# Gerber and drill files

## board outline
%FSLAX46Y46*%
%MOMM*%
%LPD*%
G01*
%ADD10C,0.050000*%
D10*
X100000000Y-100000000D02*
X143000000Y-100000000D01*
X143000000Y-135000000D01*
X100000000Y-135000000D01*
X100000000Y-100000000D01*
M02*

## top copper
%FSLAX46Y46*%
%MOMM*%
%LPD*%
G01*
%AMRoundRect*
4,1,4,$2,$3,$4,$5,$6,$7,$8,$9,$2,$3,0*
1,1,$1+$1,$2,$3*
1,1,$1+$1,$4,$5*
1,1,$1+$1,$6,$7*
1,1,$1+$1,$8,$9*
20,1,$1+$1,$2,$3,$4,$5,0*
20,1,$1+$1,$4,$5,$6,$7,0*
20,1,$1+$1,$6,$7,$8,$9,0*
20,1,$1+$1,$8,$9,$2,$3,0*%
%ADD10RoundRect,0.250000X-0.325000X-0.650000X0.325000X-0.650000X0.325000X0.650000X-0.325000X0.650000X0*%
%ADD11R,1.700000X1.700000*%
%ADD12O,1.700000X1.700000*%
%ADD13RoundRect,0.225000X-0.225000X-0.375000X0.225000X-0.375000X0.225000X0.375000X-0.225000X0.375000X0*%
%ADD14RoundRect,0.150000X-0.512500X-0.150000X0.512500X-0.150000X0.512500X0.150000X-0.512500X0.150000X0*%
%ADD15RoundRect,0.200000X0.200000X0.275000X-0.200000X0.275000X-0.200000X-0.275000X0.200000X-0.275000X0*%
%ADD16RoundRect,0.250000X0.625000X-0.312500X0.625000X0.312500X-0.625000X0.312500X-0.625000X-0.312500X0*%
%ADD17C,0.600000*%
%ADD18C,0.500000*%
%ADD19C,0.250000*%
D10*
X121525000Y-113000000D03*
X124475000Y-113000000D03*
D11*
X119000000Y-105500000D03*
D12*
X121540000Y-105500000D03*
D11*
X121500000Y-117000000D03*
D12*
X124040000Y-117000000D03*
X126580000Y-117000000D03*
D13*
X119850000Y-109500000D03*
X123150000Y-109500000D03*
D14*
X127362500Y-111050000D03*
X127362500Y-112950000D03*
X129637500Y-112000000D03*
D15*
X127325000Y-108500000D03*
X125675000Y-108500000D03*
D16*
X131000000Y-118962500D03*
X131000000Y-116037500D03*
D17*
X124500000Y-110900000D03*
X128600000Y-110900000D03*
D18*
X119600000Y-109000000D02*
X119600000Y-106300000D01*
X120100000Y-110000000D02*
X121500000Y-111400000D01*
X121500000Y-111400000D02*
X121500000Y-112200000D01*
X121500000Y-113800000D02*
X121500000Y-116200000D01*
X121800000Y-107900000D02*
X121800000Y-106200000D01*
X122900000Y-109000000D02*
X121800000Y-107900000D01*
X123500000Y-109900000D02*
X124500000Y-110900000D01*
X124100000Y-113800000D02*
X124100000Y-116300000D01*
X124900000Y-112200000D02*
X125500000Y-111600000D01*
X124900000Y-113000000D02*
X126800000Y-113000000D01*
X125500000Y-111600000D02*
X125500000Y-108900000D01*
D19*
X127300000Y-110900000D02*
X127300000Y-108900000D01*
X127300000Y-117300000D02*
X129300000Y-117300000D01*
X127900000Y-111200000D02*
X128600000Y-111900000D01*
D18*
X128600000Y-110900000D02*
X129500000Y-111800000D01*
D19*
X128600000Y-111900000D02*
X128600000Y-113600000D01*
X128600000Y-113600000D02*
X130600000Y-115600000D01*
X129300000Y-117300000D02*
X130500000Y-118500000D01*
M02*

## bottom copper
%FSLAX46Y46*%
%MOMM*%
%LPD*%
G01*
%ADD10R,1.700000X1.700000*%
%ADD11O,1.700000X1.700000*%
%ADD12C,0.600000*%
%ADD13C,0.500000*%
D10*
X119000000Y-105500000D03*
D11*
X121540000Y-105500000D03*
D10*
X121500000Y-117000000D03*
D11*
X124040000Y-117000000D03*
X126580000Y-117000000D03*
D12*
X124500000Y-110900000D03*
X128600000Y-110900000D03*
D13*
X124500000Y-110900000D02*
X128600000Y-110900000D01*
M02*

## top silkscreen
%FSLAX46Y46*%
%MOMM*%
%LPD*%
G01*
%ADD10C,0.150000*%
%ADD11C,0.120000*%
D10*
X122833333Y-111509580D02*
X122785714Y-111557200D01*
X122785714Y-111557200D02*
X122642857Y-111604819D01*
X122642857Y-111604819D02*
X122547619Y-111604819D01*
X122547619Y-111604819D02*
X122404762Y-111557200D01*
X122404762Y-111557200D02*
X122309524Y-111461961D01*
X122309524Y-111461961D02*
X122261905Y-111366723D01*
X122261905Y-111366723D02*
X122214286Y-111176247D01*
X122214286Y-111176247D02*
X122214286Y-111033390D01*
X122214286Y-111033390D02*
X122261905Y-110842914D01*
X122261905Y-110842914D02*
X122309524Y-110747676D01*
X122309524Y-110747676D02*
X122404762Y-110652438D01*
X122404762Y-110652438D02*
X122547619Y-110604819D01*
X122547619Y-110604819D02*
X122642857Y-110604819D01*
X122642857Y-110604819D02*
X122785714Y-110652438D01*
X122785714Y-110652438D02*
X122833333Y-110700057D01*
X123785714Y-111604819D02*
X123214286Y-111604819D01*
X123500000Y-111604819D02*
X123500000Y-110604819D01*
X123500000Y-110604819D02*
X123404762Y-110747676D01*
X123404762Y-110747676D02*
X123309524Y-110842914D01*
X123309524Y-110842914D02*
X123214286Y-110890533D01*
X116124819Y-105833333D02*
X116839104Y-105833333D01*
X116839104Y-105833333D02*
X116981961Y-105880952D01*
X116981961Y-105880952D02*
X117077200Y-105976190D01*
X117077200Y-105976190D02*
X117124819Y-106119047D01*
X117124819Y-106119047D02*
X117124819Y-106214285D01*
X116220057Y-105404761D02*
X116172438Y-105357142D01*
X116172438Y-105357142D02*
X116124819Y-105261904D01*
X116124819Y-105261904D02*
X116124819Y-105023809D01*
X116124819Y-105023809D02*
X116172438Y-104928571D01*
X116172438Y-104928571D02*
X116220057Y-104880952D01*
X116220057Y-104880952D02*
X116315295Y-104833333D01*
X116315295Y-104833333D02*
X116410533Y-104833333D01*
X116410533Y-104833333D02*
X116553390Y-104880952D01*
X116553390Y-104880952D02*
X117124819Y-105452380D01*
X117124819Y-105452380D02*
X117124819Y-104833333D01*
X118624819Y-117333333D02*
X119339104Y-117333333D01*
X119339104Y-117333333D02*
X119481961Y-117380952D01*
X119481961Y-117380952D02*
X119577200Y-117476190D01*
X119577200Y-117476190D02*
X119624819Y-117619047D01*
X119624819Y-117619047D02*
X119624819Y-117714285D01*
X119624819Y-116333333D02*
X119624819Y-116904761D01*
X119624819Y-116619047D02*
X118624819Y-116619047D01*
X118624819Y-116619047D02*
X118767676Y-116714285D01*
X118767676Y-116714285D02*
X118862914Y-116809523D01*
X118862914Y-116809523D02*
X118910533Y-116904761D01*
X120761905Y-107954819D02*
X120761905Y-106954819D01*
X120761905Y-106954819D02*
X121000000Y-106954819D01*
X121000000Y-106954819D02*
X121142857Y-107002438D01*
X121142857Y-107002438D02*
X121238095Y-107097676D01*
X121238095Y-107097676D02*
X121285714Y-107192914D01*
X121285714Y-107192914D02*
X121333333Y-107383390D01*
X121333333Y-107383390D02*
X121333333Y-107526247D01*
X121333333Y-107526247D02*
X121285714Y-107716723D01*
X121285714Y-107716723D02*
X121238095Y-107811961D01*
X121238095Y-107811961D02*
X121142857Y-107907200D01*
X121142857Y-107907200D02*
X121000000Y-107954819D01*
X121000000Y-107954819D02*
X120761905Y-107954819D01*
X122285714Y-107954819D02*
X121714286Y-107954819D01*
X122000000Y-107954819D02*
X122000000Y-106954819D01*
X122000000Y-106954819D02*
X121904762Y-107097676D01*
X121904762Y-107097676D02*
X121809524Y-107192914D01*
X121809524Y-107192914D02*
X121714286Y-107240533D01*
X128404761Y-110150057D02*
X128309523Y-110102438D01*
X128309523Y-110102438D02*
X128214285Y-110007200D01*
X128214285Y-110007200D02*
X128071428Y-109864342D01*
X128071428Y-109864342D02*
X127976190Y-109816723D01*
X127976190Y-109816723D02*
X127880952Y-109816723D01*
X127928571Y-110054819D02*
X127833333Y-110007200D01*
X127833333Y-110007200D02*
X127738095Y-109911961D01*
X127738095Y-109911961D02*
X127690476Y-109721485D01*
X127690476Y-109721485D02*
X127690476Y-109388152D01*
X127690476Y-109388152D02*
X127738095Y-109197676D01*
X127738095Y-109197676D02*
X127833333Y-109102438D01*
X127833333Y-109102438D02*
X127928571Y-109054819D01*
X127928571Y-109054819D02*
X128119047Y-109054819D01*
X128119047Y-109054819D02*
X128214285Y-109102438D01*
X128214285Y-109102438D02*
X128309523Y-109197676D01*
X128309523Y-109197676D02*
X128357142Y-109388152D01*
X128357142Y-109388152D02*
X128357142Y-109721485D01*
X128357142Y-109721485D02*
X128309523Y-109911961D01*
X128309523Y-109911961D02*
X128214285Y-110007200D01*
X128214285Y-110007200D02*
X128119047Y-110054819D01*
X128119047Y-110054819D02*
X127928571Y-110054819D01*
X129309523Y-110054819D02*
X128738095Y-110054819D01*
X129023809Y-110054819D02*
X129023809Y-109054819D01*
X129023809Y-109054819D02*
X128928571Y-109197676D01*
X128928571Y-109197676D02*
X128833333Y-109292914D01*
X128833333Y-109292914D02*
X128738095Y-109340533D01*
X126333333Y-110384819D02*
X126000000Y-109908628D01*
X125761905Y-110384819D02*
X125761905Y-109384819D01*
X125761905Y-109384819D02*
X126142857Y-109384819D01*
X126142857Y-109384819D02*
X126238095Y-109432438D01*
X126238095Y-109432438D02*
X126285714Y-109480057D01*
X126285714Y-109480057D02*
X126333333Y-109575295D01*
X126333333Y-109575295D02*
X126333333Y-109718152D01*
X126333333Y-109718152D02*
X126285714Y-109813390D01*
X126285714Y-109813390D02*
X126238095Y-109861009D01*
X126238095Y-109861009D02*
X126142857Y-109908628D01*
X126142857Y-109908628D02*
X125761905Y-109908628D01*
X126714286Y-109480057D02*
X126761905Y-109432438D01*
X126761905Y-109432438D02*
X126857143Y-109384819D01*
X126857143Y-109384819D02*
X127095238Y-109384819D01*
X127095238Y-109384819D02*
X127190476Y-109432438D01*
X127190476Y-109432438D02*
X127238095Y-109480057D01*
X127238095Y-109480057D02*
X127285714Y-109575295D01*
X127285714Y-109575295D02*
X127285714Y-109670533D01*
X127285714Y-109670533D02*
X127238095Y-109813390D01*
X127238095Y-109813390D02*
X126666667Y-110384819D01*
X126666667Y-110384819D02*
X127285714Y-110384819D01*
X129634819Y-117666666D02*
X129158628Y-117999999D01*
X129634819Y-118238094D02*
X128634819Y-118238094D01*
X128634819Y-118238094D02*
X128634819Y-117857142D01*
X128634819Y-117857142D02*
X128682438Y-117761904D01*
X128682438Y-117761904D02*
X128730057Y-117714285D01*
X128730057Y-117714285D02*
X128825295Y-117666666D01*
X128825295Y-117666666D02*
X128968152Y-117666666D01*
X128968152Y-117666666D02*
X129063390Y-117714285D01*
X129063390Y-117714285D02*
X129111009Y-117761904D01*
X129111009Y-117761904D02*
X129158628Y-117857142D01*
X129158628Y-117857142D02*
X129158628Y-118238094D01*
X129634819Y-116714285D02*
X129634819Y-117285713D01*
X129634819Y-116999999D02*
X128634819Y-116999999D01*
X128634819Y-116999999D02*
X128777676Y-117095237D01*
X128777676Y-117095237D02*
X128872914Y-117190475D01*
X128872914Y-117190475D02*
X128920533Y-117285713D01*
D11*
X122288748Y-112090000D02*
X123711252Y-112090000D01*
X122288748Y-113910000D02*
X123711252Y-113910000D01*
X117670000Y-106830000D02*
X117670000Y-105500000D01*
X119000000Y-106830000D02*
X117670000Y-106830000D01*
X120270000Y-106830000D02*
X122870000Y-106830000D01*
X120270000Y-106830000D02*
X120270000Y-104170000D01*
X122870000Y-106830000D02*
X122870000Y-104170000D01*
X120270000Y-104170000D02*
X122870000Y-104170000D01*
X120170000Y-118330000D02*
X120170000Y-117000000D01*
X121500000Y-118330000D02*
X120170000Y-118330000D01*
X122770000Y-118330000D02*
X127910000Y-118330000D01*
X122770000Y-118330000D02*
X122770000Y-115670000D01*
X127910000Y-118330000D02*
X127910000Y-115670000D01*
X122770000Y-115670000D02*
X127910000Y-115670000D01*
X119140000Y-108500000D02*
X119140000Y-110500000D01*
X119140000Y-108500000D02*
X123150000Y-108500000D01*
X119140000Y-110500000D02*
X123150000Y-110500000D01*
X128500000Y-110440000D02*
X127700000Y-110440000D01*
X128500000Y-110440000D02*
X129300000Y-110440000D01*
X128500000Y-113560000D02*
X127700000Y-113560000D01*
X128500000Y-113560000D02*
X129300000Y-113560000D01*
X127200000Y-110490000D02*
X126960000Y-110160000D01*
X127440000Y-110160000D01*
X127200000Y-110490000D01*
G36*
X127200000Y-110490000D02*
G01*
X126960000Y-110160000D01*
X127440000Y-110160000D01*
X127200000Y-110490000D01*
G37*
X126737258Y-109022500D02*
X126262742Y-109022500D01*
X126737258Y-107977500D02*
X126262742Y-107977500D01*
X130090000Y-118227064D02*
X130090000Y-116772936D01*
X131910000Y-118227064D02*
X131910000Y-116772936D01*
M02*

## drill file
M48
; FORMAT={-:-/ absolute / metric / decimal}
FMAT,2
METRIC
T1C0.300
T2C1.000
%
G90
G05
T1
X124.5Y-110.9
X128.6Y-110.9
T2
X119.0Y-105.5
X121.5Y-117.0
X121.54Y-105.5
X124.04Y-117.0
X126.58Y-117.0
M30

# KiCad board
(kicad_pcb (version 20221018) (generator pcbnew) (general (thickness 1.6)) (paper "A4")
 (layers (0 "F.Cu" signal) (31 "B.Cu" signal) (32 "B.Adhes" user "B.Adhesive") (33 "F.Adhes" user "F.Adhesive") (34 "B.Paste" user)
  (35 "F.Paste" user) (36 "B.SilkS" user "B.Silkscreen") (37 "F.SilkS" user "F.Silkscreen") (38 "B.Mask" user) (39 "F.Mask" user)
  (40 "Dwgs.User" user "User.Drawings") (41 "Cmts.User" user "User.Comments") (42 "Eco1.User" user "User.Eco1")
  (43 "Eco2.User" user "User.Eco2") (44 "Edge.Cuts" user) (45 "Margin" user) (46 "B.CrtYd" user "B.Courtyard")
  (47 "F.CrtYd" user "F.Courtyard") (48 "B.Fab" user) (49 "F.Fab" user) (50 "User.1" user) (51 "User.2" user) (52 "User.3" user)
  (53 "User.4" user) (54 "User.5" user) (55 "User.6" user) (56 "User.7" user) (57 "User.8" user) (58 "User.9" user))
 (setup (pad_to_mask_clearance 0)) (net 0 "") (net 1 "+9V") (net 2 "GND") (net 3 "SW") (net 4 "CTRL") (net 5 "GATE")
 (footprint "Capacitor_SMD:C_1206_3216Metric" (layer "F.Cu") (at 123 113)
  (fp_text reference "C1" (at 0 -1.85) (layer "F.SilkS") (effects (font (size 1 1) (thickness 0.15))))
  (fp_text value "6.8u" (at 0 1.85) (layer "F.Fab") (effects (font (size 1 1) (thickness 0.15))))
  (fp_line (start -0.711252 -0.91) (end 0.711252 -0.91) (stroke (width 0.12) (type solid)) (layer "F.SilkS"))
  (fp_line (start -0.711252 0.91) (end 0.711252 0.91) (stroke (width 0.12) (type solid)) (layer "F.SilkS"))
  (pad "1" smd roundrect (at -1.475 0) (size 1.15 1.8) (layers "F.Cu" "F.Paste" "F.Mask") (roundrect_rratio 0.217391) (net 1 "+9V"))
  (pad "2" smd roundrect (at 1.475 0) (size 1.15 1.8) (layers "F.Cu" "F.Paste" "F.Mask") (roundrect_rratio 0.217391) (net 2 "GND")))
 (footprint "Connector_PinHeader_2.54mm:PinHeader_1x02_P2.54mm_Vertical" (layer "F.Cu") (at 119 105.5 90)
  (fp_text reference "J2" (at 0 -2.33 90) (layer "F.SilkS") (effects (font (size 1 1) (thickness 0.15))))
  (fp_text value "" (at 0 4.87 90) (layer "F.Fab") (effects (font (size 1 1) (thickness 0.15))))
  (fp_line (start -1.33 -1.33) (end 0 -1.33) (stroke (width 0.12) (type solid)) (layer "F.SilkS"))
  (fp_line (start -1.33 0) (end -1.33 -1.33) (stroke (width 0.12) (type solid)) (layer "F.SilkS"))
  (fp_line (start -1.33 1.27) (end -1.33 3.87) (stroke (width 0.12) (type solid)) (layer "F.SilkS"))
  (fp_line (start -1.33 1.27) (end 1.33 1.27) (stroke (width 0.12) (type solid)) (layer "F.SilkS"))
  (fp_line (start -1.33 3.87) (end 1.33 3.87) (stroke (width 0.12) (type solid)) (layer "F.SilkS"))
  (fp_line (start 1.33 1.27) (end 1.33 3.87) (stroke (width 0.12) (type solid)) (layer "F.SilkS"))
  (pad "1" thru_hole rect (at 0 0 90) (size 1.7 1.7) (drill 1) (layers "*.Cu" "*.Mask") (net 1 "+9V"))
  (pad "2" thru_hole oval (at 0 2.54 90) (size 1.7 1.7) (drill 1) (layers "*.Cu" "*.Mask") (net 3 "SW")))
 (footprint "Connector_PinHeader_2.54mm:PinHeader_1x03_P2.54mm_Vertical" (layer "F.Cu") (at 121.5 117 90)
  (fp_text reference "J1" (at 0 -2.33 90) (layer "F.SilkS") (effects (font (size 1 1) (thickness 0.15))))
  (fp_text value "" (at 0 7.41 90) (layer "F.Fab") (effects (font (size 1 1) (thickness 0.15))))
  (fp_line (start -1.33 -1.33) (end 0 -1.33) (stroke (width 0.12) (type solid)) (layer "F.SilkS"))
  (fp_line (start -1.33 0) (end -1.33 -1.33) (stroke (width 0.12) (type solid)) (layer "F.SilkS"))
  (fp_line (start -1.33 1.27) (end -1.33 6.41) (stroke (width 0.12) (type solid)) (layer "F.SilkS"))
  (fp_line (start -1.33 1.27) (end 1.33 1.27) (stroke (width 0.12) (type solid)) (layer "F.SilkS"))
  (fp_line (start -1.33 6.41) (end 1.33 6.41) (stroke (width 0.12) (type solid)) (layer "F.SilkS"))
  (fp_line (start 1.33 1.27) (end 1.33 6.41) (stroke (width 0.12) (type solid)) (layer "F.SilkS"))
  (pad "1" thru_hole rect (at 0 0 90) (size 1.7 1.7) (drill 1) (layers "*.Cu" "*.Mask") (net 1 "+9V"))
  (pad "2" thru_hole oval (at 0 2.54 90) (size 1.7 1.7) (drill 1) (layers "*.Cu" "*.Mask") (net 2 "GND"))
  (pad "3" thru_hole oval (at 0 5.08 90) (size 1.7 1.7) (drill 1) (layers "*.Cu" "*.Mask") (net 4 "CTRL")))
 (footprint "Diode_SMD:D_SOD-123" (layer "F.Cu") (at 121.5 109.5)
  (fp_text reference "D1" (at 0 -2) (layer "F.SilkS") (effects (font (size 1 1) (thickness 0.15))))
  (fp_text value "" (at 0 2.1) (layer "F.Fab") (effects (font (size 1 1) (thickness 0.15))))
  (fp_line (start -2.36 -1) (end -2.36 1) (stroke (width 0.12) (type solid)) (layer "F.SilkS"))
  (fp_line (start -2.36 -1) (end 1.65 -1) (stroke (width 0.12) (type solid)) (layer "F.SilkS"))
  (fp_line (start -2.36 1) (end 1.65 1) (stroke (width 0.12) (type solid)) (layer "F.SilkS"))
  (pad "1" smd roundrect (at -1.65 0) (size 0.9 1.2) (layers "F.Cu" "F.Paste" "F.Mask") (roundrect_rratio 0.25) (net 1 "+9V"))
  (pad "2" smd roundrect (at 1.65 0) (size 0.9 1.2) (layers "F.Cu" "F.Paste" "F.Mask") (roundrect_rratio 0.25) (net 3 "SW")))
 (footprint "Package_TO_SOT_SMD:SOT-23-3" (layer "F.Cu") (at 128.5 112)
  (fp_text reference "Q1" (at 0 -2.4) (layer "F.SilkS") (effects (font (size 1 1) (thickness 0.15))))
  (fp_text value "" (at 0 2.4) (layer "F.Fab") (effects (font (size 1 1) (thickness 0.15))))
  (fp_line (start 0 -1.56) (end -0.8 -1.56) (stroke (width 0.12) (type solid)) (layer "F.SilkS"))
  (fp_line (start 0 -1.56) (end 0.8 -1.56) (stroke (width 0.12) (type solid)) (layer "F.SilkS"))
  (fp_line (start 0 1.56) (end -0.8 1.56) (stroke (width 0.12) (type solid)) (layer "F.SilkS"))
  (fp_line (start 0 1.56) (end 0.8 1.56) (stroke (width 0.12) (type solid)) (layer "F.SilkS"))
  (fp_poly
   (pts (xy -1.3 -1.51) (xy -1.54 -1.84) (xy -1.06 -1.84) (xy -1.3 -1.51)) (stroke (width 0.12) (type solid)) (fill solid) (layer "F.SilkS"))
  (pad "1" smd roundrect (at -1.1375 -0.95) (size 1.325 0.6) (layers "F.Cu" "F.Paste" "F.Mask") (roundrect_rratio 0.25) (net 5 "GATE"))
  (pad "2" smd roundrect (at -1.1375 0.95) (size 1.325 0.6) (layers "F.Cu" "F.Paste" "F.Mask") (roundrect_rratio 0.25) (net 2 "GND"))
  (pad "3" smd roundrect (at 1.1375 0) (size 1.325 0.6) (layers "F.Cu" "F.Paste" "F.Mask") (roundrect_rratio 0.25) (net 3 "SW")))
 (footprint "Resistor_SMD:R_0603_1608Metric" (layer "F.Cu") (at 126.5 108.5 180)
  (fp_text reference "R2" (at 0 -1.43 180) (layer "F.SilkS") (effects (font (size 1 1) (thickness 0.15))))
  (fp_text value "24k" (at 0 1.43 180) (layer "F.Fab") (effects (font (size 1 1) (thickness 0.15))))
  (fp_line (start -0.237258 -0.5225) (end 0.237258 -0.5225) (stroke (width 0.12) (type solid)) (layer "F.SilkS"))
  (fp_line (start -0.237258 0.5225) (end 0.237258 0.5225) (stroke (width 0.12) (type solid)) (layer "F.SilkS"))
  (pad "1" smd roundrect (at -0.825 0 180) (size 0.8 0.95) (layers "F.Cu" "F.Paste" "F.Mask") (roundrect_rratio 0.25) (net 5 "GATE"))
  (pad "2" smd roundrect (at 0.825 0 180) (size 0.8 0.95) (layers "F.Cu" "F.Paste" "F.Mask") (roundrect_rratio 0.25) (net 2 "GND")))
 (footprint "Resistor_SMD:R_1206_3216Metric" (layer "F.Cu") (at 131 117.5 90)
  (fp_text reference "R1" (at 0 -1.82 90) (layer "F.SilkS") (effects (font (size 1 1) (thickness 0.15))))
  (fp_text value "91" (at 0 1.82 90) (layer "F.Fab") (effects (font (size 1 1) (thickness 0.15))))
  (fp_line (start -0.727064 -0.91) (end 0.727064 -0.91) (stroke (width 0.12) (type solid)) (layer "F.SilkS"))
  (fp_line (start -0.727064 0.91) (end 0.727064 0.91) (stroke (width 0.12) (type solid)) (layer "F.SilkS"))
  (pad "1" smd roundrect (at -1.4625 0 90) (size 1.125 1.75) (layers "F.Cu" "F.Paste" "F.Mask") (roundrect_rratio 0.222222) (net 4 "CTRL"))
  (pad "2" smd roundrect (at 1.4625 0 90) (size 1.125 1.75) (layers "F.Cu" "F.Paste" "F.Mask") (roundrect_rratio 0.222222) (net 5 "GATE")))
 (gr_rect (start 100 100) (end 143 135) (stroke (width 0.05) (type default)) (fill none) (layer "Edge.Cuts"))
 (segment (start 119.6 109) (end 119.6 106.3) (width 0.5) (layer "F.Cu") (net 1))
 (segment (start 120.1 110) (end 121.5 111.4) (width 0.5) (layer "F.Cu") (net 1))
 (segment (start 121.5 111.4) (end 121.5 112.2) (width 0.5) (layer "F.Cu") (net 1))
 (segment (start 121.5 113.8) (end 121.5 116.2) (width 0.5) (layer "F.Cu") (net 1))
 (segment (start 121.8 107.9) (end 121.8 106.2) (width 0.5) (layer "F.Cu") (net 3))
 (segment (start 122.9 109) (end 121.8 107.9) (width 0.5) (layer "F.Cu") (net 3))
 (segment (start 123.5 109.9) (end 124.5 110.9) (width 0.5) (layer "F.Cu") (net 3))
 (segment (start 124.1 113.8) (end 124.1 116.3) (width 0.5) (layer "F.Cu") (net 2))
 (segment (start 124.9 112.2) (end 125.5 111.6) (width 0.5) (layer "F.Cu") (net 2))
 (segment (start 124.9 113) (end 126.8 113) (width 0.5) (layer "F.Cu") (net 2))
 (segment (start 125.5 111.6) (end 125.5 108.9) (width 0.5) (layer "F.Cu") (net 2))
 (segment (start 127.3 110.9) (end 127.3 108.9) (width 0.25) (layer "F.Cu") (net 5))
 (segment (start 127.3 117.3) (end 129.3 117.3) (width 0.25) (layer "F.Cu") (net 4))
 (segment (start 127.9 111.2) (end 128.6 111.9) (width 0.25) (layer "F.Cu") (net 5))
 (segment (start 128.6 110.9) (end 129.5 111.8) (width 0.5) (layer "F.Cu") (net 3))
 (segment (start 128.6 111.9) (end 128.6 113.6) (width 0.25) (layer "F.Cu") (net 5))
 (segment (start 128.6 113.6) (end 130.6 115.6) (width 0.25) (layer "F.Cu") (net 5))
 (segment (start 129.3 117.3) (end 130.5 118.5) (width 0.25) (layer "F.Cu") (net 4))
 (via (at 124.5 110.9) (size 0.6) (drill 0.3) (layers "F.Cu" "B.Cu") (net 3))
 (via (at 128.6 110.9) (size 0.6) (drill 0.3) (layers "F.Cu" "B.Cu") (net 3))
 (segment (start 124.5 110.9) (end 128.6 110.9) (width 0.5) (layer "B.Cu") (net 3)))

